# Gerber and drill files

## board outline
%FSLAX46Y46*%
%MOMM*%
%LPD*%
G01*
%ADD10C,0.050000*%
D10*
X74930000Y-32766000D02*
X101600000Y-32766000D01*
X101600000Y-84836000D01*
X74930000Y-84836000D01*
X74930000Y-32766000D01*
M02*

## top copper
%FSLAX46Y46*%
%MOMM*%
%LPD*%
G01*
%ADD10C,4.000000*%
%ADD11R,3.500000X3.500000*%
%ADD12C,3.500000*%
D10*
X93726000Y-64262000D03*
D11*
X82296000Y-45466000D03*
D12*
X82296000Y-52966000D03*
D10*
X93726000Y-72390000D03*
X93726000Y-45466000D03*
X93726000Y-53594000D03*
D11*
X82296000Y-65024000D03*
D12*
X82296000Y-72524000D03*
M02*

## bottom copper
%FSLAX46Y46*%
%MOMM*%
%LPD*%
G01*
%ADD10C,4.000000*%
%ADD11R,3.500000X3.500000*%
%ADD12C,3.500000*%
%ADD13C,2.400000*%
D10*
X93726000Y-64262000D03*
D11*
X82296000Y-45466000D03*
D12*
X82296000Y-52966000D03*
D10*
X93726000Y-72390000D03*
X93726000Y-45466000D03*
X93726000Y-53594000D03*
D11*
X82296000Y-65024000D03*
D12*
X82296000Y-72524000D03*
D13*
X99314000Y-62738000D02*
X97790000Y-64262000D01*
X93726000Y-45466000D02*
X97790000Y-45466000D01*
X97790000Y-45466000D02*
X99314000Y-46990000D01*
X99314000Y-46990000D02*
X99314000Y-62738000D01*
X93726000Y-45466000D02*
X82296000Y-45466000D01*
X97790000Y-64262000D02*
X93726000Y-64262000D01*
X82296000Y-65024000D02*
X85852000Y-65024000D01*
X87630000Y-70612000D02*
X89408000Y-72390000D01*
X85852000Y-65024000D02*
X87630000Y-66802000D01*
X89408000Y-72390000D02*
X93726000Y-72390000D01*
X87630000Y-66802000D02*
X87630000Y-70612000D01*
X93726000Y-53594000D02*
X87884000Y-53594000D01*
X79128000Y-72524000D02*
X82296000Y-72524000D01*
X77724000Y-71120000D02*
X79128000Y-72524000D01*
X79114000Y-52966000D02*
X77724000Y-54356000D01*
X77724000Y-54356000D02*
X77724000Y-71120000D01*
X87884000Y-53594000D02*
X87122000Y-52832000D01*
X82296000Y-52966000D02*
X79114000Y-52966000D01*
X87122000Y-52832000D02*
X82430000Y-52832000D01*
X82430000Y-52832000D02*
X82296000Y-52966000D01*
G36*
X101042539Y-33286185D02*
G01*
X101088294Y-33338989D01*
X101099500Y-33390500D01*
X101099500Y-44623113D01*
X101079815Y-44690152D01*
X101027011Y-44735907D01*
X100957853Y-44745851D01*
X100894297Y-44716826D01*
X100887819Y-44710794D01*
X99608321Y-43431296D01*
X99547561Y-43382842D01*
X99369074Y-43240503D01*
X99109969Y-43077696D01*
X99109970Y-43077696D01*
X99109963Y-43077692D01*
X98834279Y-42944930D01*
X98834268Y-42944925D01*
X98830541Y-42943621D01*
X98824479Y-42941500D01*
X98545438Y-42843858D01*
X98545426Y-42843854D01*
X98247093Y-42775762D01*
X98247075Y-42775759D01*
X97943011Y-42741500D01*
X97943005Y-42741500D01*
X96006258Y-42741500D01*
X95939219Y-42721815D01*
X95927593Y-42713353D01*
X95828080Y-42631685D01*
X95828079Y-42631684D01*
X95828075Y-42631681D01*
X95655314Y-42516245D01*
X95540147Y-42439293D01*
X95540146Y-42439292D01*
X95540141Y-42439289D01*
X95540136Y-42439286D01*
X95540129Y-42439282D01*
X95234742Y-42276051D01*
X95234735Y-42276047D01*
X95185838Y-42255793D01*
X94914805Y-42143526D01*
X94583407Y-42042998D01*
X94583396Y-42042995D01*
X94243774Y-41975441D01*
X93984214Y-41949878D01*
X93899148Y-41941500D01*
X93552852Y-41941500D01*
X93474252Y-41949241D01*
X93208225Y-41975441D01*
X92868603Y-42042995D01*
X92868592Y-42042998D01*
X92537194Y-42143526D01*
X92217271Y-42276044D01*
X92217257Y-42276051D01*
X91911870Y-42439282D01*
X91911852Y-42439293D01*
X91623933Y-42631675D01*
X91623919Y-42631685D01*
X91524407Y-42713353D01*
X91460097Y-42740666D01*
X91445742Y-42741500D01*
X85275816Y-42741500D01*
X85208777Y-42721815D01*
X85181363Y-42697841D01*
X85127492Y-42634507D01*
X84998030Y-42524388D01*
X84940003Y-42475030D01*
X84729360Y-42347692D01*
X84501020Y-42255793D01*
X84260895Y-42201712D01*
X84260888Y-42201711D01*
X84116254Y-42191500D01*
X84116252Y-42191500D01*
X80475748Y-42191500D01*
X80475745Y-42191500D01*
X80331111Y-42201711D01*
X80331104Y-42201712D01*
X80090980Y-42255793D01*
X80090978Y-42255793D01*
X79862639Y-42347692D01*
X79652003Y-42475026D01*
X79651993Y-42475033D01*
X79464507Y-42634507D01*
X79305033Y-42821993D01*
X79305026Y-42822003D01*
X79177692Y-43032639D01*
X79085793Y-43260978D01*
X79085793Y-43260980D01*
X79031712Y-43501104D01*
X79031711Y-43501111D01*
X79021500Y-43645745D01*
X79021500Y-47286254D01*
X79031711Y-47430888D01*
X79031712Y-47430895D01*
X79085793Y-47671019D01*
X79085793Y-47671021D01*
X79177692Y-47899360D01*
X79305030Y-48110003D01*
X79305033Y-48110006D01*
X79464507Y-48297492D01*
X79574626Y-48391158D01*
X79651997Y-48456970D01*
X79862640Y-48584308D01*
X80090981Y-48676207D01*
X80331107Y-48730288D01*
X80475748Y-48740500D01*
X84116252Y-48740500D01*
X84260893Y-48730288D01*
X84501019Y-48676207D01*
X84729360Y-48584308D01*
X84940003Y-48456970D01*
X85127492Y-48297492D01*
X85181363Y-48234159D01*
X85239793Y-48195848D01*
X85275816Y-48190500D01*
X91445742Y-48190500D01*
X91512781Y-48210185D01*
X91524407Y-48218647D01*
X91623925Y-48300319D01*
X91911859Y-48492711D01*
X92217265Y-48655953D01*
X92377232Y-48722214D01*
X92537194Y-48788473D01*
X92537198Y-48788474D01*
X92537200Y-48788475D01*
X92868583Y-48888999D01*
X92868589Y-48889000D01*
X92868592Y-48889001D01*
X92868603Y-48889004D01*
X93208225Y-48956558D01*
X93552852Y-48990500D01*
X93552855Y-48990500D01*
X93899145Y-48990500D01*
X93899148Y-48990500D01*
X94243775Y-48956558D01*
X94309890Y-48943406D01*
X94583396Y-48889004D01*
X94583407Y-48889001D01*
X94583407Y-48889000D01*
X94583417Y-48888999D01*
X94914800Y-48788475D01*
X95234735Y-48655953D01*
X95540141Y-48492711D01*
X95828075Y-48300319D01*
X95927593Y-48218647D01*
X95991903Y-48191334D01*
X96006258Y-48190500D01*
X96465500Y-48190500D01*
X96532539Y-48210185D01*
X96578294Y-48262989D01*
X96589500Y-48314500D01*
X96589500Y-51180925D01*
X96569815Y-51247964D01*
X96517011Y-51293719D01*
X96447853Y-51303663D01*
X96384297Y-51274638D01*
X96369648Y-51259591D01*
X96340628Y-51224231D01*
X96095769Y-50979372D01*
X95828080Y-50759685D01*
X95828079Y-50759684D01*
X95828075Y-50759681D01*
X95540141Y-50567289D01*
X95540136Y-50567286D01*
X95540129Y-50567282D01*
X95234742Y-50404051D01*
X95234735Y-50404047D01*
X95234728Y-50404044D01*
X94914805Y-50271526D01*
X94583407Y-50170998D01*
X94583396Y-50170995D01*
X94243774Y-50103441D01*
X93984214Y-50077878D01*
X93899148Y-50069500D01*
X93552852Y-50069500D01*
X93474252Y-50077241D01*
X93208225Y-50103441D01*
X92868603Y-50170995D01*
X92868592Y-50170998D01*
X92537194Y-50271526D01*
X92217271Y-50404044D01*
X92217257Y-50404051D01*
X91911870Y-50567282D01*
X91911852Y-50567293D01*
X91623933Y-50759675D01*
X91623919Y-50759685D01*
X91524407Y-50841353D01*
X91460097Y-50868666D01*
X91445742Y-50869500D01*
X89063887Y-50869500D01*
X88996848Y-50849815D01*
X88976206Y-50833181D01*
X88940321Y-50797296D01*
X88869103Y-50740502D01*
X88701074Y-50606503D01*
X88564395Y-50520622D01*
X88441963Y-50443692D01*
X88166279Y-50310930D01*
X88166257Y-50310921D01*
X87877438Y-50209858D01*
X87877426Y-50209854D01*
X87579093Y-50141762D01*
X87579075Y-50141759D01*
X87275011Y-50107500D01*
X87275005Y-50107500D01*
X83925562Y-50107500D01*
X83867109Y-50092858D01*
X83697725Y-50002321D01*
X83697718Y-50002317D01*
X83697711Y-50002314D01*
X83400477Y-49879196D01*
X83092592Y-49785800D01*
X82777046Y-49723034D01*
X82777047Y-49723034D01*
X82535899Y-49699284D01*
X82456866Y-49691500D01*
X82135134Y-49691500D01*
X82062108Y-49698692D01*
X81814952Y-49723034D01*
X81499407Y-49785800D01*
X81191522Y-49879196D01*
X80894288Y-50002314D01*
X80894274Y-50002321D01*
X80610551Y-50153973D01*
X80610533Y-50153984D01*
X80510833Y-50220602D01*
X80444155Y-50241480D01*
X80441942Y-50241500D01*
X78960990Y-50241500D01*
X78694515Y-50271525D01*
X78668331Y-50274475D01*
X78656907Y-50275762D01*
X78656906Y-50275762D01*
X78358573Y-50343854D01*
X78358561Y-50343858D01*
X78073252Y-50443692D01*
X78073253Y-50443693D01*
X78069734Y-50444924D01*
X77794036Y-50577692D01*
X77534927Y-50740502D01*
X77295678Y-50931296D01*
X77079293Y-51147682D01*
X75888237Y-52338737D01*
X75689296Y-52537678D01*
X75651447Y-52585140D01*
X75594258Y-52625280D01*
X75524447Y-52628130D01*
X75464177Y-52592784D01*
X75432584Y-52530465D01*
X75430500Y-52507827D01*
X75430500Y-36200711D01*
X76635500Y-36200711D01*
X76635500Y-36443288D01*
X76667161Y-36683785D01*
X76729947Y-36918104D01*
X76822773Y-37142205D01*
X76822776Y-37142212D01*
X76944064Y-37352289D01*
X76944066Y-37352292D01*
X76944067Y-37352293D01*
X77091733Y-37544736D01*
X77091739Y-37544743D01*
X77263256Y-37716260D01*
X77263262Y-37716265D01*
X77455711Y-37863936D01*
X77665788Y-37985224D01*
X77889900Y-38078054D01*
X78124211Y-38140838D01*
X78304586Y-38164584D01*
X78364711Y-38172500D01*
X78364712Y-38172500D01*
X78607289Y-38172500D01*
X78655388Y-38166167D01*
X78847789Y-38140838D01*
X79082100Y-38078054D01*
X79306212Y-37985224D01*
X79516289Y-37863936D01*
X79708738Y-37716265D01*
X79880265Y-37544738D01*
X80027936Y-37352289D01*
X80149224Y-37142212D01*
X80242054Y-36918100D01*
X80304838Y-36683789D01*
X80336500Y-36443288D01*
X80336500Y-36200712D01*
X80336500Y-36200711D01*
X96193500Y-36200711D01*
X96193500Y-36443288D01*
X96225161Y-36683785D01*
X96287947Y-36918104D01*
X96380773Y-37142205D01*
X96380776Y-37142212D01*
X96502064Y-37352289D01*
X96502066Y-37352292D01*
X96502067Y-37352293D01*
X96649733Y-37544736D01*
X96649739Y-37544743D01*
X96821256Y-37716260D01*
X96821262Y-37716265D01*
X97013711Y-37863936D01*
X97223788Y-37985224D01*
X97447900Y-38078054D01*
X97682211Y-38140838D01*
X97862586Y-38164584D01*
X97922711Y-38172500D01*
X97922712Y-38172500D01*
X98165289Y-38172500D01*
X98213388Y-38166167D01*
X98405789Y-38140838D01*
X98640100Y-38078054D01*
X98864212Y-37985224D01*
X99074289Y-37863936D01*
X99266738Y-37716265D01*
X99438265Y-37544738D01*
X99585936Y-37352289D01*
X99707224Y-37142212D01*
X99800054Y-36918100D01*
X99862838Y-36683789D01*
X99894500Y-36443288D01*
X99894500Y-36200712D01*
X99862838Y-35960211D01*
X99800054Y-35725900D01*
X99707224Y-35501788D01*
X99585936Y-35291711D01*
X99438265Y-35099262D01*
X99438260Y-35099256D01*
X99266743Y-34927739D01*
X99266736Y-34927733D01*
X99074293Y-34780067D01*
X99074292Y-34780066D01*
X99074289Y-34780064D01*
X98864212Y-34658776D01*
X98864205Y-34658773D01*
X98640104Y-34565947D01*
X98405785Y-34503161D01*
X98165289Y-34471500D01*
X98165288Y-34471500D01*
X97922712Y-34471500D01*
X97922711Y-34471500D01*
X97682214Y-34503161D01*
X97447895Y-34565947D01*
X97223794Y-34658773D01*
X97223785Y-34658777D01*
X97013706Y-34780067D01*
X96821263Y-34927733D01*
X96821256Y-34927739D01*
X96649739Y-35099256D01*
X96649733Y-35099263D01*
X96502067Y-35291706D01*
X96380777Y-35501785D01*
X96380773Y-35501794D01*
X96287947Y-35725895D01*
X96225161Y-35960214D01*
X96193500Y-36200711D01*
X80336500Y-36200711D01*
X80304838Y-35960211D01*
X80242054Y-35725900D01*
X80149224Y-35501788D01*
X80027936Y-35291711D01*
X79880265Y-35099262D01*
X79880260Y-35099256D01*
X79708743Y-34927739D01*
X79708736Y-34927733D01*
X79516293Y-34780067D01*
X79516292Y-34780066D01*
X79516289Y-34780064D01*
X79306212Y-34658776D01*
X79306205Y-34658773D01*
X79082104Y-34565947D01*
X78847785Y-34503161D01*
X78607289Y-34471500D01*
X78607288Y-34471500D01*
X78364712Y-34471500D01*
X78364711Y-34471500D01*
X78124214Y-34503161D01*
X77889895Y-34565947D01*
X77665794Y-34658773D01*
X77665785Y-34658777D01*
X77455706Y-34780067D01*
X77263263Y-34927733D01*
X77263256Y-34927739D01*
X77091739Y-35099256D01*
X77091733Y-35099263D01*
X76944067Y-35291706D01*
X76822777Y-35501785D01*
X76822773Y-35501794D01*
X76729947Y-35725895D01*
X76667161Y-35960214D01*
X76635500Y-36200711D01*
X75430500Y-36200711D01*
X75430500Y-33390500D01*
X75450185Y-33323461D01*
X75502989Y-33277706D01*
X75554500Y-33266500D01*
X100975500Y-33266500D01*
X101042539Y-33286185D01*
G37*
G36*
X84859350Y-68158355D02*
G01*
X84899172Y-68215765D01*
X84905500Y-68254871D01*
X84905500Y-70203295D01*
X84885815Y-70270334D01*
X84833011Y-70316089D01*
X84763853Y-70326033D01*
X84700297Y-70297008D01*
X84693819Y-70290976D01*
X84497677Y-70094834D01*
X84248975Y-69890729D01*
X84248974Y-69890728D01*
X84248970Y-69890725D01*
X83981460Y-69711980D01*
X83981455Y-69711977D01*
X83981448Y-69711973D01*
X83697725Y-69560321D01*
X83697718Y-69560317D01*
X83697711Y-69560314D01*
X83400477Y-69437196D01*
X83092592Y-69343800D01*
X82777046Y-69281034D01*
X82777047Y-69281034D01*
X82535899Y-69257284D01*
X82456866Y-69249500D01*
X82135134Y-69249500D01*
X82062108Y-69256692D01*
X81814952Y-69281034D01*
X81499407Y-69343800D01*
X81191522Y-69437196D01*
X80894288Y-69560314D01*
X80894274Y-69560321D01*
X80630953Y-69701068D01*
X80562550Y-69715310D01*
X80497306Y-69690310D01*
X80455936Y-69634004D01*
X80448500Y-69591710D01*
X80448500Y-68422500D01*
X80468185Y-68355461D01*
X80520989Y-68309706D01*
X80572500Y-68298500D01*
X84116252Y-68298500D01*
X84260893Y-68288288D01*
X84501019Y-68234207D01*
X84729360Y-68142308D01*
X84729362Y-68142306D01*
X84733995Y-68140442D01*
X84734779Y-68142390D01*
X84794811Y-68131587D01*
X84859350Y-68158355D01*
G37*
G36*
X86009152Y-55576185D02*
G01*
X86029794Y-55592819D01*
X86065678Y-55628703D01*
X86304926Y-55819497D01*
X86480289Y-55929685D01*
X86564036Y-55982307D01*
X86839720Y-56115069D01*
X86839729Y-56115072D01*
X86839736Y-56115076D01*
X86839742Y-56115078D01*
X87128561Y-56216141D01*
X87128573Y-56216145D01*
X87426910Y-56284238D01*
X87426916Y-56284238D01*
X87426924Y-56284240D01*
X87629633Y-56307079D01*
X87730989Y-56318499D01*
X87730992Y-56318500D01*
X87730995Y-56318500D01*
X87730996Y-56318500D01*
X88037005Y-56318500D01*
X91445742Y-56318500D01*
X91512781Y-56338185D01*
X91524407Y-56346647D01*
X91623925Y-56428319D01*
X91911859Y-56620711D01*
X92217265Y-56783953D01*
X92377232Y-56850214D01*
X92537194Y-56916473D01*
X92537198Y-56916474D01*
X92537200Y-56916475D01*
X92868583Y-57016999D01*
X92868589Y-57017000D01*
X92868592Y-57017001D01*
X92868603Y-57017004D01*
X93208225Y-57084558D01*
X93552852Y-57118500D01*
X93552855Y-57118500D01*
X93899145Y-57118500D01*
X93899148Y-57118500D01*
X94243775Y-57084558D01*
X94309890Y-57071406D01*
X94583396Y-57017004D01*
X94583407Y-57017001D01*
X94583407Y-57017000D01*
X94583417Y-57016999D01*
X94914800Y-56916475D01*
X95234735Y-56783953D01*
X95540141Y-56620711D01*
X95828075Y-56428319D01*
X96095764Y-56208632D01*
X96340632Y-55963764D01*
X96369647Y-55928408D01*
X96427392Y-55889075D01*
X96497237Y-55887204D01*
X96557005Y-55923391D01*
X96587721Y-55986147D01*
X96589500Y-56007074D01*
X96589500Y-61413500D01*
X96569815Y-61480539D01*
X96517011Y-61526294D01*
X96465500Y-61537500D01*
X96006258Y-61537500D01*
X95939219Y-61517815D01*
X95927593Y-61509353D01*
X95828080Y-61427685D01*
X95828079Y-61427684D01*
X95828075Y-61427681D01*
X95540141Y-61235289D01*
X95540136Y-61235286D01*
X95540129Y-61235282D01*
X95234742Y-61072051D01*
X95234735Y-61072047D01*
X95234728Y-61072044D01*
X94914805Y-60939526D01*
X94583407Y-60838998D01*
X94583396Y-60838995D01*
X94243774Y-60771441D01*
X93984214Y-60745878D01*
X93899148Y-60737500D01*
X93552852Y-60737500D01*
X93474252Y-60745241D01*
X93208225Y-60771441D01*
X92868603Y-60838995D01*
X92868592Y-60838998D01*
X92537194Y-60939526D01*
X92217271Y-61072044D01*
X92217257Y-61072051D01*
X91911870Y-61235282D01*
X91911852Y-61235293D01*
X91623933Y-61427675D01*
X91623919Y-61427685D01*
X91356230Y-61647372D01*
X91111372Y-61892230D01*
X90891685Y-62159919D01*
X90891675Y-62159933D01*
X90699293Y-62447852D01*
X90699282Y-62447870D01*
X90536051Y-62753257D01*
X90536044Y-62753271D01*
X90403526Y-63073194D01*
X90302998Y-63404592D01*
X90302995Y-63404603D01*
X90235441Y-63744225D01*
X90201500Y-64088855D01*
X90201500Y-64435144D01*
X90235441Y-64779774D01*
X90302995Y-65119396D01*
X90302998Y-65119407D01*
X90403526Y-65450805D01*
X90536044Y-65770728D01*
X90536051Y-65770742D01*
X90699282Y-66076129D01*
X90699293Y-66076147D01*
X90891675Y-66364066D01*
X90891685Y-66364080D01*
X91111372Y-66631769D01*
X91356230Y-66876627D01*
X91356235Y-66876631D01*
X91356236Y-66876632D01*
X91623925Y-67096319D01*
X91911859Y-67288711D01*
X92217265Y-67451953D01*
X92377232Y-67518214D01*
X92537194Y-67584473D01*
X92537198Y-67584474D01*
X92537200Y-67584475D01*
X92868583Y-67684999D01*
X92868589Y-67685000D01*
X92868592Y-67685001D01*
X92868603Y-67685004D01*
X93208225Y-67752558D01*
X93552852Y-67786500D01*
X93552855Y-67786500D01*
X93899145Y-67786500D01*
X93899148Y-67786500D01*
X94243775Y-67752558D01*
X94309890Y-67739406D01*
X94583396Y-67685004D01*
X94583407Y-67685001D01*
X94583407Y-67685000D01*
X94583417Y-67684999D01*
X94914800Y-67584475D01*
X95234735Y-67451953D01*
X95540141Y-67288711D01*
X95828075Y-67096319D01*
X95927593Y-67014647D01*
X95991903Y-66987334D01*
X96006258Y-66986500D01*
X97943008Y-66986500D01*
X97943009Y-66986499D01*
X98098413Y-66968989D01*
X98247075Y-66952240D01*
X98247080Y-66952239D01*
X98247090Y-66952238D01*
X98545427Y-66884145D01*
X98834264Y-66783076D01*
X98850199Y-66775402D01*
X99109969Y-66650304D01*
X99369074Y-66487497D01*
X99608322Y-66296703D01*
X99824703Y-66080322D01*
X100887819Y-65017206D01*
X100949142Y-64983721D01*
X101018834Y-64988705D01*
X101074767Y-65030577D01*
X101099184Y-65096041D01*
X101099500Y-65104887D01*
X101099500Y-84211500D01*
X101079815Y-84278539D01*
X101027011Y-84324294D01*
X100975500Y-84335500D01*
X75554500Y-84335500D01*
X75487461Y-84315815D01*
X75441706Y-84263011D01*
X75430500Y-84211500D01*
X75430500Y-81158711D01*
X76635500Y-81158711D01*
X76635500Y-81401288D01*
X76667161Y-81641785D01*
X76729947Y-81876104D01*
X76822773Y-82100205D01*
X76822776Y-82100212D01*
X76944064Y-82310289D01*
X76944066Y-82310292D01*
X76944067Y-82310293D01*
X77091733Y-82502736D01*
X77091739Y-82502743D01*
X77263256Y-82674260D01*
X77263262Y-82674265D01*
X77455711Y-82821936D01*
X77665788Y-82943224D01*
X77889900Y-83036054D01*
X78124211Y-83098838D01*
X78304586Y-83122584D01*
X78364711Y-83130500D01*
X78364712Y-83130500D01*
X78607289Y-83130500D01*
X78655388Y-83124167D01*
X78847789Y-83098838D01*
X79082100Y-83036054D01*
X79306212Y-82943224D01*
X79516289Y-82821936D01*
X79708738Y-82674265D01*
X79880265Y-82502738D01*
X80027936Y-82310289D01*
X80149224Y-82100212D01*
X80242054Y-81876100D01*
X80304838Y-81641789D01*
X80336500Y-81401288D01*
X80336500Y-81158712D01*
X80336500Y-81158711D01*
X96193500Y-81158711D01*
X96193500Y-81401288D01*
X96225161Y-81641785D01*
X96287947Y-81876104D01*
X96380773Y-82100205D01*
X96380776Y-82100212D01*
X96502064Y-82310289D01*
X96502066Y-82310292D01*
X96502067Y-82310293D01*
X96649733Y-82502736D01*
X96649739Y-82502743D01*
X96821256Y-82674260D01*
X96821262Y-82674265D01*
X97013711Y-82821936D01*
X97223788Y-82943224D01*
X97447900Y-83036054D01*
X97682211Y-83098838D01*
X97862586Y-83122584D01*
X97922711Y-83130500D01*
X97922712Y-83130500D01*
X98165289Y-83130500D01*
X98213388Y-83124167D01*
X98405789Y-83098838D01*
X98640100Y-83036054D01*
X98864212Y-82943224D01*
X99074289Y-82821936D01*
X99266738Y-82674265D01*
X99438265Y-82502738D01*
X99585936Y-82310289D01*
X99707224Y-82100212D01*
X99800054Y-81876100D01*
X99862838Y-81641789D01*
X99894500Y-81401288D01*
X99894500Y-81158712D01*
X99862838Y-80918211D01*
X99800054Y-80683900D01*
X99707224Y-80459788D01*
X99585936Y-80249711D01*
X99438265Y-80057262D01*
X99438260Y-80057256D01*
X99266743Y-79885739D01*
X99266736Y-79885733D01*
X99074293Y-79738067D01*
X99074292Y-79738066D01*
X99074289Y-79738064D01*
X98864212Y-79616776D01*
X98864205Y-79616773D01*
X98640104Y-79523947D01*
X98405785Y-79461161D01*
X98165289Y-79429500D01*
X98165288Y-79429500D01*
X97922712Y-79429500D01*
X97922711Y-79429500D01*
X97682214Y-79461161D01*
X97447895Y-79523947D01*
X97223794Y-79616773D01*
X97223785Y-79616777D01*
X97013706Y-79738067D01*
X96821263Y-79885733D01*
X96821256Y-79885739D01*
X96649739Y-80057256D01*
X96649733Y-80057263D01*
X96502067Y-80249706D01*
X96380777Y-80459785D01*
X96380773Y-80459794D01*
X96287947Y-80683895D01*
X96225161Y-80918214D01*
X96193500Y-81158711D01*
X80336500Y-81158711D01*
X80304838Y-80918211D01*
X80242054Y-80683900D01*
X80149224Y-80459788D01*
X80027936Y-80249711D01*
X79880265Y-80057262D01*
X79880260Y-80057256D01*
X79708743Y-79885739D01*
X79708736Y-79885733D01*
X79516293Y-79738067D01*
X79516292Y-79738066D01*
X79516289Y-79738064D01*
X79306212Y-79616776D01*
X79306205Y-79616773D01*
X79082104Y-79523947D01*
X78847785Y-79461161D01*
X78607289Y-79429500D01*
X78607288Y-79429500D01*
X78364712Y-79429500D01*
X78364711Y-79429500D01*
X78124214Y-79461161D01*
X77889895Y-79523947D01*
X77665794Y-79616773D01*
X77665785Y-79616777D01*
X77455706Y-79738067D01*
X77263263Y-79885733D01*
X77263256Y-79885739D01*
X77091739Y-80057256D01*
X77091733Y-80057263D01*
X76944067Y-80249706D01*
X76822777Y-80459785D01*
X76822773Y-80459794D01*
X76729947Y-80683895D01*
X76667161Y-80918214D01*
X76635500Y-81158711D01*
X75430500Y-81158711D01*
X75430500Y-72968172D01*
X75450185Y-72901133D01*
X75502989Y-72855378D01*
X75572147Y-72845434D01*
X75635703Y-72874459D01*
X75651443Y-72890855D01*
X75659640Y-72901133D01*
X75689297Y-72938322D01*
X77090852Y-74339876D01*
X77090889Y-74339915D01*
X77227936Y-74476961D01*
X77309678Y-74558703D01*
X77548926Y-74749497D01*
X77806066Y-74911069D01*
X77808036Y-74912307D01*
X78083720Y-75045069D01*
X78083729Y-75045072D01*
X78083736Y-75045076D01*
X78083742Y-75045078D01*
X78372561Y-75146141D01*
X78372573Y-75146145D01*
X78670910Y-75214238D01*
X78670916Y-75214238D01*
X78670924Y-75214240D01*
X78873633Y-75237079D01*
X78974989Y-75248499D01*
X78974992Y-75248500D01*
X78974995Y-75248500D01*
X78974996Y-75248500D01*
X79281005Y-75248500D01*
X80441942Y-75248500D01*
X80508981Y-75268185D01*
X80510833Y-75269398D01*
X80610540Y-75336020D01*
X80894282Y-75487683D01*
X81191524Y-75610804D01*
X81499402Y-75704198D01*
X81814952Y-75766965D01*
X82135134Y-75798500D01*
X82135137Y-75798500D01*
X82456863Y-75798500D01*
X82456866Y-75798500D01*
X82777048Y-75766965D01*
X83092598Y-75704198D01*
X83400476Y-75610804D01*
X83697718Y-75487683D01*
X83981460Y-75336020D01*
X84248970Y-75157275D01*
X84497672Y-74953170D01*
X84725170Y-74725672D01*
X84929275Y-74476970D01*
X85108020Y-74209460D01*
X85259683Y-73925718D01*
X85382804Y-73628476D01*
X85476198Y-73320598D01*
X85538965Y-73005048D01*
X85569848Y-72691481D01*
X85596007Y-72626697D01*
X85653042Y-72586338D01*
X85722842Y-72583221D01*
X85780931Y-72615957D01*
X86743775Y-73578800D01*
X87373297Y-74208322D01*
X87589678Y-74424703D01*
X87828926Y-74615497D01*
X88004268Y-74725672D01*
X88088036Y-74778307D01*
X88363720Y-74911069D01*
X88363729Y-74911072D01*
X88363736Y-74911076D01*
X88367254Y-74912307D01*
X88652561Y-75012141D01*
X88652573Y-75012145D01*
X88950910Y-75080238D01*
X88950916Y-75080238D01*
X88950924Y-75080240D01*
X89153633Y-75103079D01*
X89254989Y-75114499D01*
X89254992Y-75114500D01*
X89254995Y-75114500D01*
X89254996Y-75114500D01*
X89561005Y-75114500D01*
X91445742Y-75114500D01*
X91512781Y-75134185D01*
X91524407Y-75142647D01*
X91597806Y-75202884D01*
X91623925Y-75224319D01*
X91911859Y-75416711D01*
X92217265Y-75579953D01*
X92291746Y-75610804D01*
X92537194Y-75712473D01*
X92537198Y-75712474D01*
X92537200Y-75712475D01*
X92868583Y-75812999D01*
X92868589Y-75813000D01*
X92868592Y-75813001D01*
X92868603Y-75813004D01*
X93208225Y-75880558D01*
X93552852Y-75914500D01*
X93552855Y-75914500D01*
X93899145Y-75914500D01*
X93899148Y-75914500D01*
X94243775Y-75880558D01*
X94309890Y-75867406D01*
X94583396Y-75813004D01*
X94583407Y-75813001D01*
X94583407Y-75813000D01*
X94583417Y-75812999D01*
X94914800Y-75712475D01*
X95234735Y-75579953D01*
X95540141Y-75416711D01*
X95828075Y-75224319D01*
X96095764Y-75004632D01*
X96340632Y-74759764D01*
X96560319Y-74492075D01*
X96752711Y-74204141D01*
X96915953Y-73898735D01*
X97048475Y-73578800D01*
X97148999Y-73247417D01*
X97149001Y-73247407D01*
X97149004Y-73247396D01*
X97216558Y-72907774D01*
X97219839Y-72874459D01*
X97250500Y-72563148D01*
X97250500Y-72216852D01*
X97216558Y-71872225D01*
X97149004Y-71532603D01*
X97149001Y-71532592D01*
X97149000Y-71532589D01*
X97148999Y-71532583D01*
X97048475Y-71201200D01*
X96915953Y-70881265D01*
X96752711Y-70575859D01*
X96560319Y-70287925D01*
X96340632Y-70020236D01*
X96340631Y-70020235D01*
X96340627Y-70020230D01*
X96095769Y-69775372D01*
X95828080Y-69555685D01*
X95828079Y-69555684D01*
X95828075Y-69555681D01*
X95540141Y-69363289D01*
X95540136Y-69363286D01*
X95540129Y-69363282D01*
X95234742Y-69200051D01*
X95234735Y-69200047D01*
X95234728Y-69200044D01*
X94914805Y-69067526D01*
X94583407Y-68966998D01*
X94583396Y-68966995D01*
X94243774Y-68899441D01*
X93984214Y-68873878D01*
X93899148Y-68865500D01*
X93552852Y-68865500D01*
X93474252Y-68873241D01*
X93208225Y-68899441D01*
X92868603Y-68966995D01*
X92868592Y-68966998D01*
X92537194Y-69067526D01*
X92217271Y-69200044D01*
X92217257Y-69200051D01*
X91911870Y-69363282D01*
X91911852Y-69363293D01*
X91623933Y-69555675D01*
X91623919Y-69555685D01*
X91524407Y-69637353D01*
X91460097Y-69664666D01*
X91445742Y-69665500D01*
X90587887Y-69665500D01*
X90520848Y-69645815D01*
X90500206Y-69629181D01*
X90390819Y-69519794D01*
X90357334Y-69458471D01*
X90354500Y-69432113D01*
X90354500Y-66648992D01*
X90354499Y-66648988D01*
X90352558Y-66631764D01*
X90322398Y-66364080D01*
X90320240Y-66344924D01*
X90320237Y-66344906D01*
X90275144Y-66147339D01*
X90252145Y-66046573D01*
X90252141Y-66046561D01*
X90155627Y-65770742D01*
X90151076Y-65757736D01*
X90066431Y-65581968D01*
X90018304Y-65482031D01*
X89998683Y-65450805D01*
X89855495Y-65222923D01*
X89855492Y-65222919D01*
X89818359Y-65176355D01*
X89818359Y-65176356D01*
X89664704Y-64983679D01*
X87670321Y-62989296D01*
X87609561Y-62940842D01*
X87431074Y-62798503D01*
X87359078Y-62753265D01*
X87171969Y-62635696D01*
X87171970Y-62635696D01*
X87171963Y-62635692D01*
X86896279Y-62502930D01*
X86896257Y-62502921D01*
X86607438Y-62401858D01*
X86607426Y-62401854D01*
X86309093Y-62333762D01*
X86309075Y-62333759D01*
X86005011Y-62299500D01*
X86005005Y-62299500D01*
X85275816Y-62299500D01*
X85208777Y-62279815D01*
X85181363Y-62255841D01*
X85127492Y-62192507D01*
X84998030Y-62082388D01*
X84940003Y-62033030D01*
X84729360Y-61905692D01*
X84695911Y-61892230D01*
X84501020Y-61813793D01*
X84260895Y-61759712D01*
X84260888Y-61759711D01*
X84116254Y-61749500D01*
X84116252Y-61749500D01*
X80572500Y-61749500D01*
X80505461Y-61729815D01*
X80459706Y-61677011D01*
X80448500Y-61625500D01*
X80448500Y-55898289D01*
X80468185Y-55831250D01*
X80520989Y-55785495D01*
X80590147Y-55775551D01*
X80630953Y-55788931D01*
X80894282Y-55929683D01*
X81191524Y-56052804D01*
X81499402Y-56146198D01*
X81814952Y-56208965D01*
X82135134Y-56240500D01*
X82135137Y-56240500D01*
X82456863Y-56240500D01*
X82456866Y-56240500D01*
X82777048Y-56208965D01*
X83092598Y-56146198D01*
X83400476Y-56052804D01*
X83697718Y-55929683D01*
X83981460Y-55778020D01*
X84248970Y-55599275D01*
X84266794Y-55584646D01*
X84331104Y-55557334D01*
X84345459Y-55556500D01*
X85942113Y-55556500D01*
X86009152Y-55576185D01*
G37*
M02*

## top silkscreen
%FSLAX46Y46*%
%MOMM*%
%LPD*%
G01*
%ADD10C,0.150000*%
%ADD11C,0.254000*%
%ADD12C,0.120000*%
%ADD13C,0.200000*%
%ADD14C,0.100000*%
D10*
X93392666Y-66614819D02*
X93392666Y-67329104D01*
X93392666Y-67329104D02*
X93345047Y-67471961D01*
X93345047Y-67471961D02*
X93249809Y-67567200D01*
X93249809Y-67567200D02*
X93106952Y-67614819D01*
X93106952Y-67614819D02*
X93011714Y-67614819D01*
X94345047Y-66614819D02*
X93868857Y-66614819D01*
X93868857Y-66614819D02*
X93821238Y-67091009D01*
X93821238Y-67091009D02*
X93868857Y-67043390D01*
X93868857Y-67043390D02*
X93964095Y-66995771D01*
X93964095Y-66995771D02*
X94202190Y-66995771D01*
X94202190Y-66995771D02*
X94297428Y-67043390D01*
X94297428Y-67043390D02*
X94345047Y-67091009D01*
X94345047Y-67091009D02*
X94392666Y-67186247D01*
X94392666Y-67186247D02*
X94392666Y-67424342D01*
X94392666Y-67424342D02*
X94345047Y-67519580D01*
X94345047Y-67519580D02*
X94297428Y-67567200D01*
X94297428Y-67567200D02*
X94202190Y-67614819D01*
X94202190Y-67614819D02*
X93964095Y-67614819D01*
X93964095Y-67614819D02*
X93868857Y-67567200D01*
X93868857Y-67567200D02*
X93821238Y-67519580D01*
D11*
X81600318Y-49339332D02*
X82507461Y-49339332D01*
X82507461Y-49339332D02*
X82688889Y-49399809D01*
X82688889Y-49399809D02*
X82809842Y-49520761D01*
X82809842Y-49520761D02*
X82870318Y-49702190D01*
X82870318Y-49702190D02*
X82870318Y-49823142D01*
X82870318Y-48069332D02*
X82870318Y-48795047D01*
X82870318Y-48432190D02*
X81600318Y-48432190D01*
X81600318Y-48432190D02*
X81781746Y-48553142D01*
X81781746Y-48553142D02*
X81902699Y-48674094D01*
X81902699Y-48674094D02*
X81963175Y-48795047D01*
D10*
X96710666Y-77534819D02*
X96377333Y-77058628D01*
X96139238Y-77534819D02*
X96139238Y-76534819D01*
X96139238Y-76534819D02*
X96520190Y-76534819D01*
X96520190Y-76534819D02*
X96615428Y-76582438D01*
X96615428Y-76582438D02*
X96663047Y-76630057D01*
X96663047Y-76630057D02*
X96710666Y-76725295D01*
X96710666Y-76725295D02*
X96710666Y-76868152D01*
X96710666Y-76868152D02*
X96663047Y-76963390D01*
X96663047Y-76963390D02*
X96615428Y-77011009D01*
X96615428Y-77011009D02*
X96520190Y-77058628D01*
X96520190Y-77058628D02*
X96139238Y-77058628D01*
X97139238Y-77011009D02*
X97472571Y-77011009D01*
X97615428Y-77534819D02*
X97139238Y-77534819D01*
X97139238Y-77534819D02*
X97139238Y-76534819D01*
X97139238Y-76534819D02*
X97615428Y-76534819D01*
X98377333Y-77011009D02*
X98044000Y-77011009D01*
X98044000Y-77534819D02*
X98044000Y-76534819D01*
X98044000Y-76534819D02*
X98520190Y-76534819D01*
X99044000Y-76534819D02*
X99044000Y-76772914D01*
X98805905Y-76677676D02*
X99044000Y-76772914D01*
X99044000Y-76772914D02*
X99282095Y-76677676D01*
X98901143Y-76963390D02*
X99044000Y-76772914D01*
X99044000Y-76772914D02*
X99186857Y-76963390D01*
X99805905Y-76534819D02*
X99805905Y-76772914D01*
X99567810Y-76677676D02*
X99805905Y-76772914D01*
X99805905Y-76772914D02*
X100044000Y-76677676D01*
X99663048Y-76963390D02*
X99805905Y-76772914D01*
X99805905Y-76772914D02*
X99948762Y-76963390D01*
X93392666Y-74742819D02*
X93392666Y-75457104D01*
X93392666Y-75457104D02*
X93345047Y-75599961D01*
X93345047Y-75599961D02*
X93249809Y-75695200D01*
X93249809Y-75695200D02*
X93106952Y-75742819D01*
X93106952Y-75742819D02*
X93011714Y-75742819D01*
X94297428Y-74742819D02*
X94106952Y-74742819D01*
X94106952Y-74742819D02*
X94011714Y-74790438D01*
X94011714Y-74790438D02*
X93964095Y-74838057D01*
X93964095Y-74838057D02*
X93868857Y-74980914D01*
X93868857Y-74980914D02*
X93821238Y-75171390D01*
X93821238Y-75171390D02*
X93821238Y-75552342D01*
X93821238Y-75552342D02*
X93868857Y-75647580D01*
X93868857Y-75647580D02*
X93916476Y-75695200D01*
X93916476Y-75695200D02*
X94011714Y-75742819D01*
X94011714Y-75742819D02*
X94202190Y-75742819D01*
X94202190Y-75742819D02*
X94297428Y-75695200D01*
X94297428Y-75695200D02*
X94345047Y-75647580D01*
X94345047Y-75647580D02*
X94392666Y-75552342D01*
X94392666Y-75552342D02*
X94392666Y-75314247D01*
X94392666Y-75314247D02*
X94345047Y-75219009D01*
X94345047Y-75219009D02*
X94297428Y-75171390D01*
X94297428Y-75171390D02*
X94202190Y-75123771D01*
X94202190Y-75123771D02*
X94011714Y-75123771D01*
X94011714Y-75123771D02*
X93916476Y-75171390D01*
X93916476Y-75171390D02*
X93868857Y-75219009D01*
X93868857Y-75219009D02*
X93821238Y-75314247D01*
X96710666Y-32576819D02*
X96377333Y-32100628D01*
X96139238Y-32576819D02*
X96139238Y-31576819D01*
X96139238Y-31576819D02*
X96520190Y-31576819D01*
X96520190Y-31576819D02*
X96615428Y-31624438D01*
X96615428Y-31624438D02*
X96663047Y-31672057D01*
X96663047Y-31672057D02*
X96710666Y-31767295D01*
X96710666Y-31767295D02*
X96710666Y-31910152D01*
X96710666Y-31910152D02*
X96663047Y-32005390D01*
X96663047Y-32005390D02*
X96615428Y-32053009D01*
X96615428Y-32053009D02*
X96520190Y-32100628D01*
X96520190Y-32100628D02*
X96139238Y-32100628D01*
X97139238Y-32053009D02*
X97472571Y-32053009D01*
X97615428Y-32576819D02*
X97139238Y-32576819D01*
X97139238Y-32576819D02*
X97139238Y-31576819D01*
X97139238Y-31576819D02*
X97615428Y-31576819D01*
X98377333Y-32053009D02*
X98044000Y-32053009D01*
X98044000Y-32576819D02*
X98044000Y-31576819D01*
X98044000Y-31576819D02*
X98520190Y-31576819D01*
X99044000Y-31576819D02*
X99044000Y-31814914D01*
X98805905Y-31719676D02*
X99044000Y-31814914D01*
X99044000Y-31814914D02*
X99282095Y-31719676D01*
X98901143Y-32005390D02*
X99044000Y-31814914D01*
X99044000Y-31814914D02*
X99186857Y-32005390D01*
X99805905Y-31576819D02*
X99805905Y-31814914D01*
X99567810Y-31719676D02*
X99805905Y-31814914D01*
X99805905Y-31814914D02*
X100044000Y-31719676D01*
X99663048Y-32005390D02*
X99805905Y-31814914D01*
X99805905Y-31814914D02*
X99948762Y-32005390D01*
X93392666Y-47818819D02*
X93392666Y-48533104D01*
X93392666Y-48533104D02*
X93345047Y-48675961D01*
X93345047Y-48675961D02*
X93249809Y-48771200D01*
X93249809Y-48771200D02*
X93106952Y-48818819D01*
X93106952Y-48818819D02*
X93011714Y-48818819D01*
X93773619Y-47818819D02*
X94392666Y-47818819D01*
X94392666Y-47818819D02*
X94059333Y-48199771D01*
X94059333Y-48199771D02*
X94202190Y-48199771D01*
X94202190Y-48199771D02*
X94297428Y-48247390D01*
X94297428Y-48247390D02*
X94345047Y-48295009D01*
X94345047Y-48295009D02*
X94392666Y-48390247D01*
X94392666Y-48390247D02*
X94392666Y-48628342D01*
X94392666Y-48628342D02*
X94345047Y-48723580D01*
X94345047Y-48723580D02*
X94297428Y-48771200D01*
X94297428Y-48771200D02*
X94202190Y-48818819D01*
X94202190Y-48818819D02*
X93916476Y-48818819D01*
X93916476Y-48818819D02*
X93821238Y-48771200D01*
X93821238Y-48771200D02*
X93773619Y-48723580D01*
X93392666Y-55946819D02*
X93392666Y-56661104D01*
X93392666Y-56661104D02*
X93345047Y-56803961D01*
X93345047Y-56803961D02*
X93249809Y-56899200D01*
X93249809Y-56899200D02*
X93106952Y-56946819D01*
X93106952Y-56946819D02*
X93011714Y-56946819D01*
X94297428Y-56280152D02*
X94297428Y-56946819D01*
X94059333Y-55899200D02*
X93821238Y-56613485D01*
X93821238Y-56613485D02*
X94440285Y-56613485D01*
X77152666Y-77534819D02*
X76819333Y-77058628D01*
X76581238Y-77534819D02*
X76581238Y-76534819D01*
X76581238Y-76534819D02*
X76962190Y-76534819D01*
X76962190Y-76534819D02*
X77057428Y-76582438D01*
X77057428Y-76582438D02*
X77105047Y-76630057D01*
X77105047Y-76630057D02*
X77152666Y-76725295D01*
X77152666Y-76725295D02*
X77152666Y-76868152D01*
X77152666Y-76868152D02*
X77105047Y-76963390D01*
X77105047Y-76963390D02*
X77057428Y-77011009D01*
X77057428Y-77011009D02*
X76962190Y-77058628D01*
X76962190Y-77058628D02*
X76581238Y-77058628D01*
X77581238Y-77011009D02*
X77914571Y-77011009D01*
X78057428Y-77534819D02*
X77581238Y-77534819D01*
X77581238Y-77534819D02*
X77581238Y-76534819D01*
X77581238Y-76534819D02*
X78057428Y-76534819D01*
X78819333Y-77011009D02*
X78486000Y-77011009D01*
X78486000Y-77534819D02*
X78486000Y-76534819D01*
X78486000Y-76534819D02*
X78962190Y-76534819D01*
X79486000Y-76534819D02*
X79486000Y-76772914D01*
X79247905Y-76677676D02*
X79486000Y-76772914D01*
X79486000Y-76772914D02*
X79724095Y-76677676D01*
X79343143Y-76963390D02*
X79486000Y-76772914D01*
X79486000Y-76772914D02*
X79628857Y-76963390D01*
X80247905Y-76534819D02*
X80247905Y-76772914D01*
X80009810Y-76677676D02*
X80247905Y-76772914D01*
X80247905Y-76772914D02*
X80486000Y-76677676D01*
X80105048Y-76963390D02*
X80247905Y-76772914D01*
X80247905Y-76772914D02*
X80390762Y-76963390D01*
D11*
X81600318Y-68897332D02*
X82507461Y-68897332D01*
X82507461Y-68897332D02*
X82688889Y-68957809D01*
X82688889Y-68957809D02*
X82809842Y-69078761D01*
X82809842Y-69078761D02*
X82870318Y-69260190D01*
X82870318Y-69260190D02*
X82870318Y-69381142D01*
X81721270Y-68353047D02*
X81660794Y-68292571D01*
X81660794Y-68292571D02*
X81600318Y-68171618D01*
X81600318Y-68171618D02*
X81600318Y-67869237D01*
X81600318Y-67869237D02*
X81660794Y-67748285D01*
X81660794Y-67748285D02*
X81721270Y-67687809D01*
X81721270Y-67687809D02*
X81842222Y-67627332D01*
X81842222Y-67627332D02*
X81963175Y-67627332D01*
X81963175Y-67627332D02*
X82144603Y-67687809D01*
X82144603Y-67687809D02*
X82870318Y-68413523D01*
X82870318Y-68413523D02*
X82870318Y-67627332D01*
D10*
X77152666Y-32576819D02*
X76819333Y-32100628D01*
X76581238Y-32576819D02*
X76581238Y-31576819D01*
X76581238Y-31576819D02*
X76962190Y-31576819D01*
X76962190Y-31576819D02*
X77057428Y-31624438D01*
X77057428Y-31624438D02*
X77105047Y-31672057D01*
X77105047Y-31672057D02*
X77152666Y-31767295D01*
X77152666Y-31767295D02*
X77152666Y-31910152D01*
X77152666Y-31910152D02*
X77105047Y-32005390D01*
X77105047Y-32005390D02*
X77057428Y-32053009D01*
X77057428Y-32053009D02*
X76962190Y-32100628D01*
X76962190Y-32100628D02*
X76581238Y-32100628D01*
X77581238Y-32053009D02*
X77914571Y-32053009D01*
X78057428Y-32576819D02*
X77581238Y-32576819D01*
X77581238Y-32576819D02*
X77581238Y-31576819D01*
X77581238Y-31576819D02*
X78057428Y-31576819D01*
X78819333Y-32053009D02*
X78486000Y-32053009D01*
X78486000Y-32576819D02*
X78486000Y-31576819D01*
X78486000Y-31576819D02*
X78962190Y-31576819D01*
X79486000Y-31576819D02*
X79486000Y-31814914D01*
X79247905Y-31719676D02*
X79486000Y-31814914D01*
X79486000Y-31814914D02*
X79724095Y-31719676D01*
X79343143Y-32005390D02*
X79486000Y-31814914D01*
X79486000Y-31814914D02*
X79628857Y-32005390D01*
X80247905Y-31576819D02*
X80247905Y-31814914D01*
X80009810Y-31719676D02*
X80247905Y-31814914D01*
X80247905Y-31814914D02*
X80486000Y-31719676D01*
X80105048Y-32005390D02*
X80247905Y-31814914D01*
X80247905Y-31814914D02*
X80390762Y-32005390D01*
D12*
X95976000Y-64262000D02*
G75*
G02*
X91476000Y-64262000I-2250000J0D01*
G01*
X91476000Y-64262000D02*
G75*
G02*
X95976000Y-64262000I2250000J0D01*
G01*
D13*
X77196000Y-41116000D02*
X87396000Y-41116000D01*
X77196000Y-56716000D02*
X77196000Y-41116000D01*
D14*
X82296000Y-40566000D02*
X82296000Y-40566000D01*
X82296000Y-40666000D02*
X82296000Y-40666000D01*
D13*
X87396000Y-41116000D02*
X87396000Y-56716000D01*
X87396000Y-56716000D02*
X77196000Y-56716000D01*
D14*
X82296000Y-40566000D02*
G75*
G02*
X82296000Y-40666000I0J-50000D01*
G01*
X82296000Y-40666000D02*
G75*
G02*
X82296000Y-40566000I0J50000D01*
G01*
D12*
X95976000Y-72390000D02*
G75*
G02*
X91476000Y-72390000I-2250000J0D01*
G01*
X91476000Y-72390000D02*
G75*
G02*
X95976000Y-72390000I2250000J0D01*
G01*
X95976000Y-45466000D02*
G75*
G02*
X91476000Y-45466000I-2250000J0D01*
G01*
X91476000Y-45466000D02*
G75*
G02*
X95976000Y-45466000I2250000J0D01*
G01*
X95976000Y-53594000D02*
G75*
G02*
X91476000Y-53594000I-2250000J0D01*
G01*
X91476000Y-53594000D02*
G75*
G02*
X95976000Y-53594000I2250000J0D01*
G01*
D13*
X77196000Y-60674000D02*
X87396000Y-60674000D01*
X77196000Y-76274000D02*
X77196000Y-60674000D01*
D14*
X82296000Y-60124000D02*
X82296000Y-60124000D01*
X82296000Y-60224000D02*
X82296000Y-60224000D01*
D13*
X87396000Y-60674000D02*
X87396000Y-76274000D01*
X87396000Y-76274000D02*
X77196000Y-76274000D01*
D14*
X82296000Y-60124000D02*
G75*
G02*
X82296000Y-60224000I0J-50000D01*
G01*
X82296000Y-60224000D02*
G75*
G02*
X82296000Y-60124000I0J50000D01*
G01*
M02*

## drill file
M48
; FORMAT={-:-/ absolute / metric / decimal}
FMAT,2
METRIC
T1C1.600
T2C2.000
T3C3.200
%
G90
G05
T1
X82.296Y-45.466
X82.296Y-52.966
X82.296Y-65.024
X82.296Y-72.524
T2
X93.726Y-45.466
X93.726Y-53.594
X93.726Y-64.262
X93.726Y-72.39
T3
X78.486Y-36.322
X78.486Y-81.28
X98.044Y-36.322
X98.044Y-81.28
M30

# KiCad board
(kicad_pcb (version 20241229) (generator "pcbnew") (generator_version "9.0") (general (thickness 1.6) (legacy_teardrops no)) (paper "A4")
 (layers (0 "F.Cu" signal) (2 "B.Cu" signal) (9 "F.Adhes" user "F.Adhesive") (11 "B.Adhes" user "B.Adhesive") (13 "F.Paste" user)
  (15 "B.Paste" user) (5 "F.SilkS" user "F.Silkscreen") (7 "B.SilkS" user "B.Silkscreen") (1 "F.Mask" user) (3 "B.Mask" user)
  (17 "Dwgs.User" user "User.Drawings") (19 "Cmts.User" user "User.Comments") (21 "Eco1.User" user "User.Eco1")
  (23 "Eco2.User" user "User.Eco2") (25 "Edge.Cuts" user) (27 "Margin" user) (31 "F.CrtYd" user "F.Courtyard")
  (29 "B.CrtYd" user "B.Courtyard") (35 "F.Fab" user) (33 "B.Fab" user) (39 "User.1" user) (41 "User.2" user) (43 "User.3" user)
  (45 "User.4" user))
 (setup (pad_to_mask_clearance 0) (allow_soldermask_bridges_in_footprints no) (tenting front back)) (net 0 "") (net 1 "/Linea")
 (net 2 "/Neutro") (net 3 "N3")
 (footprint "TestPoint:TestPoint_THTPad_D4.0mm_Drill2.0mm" (layer "F.Cu") (at 93.726 64.262 180)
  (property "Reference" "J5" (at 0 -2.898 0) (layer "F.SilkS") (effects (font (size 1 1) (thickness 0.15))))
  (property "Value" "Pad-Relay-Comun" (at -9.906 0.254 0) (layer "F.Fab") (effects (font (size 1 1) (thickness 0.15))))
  (fp_circle (center 0 0) (end 0 2.25) (stroke (width 0.12) (type solid)) (fill no) (layer "F.SilkS"))
  (pad "1" thru_hole circle (at 0 0 180) (size 4 4) (drill 2) (layers "*.Cu" "*.Mask") (remove_unused_layers no) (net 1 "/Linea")))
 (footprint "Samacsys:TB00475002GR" (layer "F.Cu") (at 82.296 45.466 -90)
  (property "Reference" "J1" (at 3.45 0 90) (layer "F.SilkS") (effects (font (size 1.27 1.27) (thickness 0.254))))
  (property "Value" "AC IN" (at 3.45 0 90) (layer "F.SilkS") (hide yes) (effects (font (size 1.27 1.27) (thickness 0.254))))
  (fp_line (start -4.35 5.1) (end -4.35 -5.1) (stroke (width 0.2) (type solid)) (layer "F.SilkS"))
  (fp_line (start 11.25 5.1) (end -4.35 5.1) (stroke (width 0.2) (type solid)) (layer "F.SilkS"))
  (fp_line (start -4.9 0) (end -4.9 0) (stroke (width 0.1) (type solid)) (layer "F.SilkS"))
  (fp_line (start -4.8 0) (end -4.8 0) (stroke (width 0.1) (type solid)) (layer "F.SilkS"))
  (fp_line (start -4.35 -5.1) (end 11.25 -5.1) (stroke (width 0.2) (type solid)) (layer "F.SilkS"))
  (fp_line (start 11.25 -5.1) (end 11.25 5.1) (stroke (width 0.2) (type solid)) (layer "F.SilkS"))
  (fp_arc (start -4.9 0) (mid -4.85 -0.05) (end -4.8 0) (stroke (width 0.1) (type solid)) (layer "F.SilkS"))
  (fp_arc (start -4.8 0) (mid -4.85 0.05) (end -4.9 0) (stroke (width 0.1) (type solid)) (layer "F.SilkS"))
  (pad "1" thru_hole rect (at 0 0 270) (size 3.5 3.5) (drill 1.6) (layers "*.Cu" "*.Mask") (remove_unused_layers no) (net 1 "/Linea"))
  (pad "2" thru_hole circle (at 7.5 0 270) (size 3.5 3.5) (drill 1.6) (layers "*.Cu" "*.Mask") (remove_unused_layers no) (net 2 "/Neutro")))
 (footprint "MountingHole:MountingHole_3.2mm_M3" (layer "F.Cu") (at 98.044 81.28)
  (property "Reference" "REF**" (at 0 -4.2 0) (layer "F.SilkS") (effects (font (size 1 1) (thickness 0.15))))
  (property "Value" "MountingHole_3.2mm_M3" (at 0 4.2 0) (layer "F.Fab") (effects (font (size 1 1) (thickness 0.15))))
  (pad "" np_thru_hole circle (at 0 0) (size 3.2 3.2) (drill 3.2) (layers "*.Cu" "*.Mask")))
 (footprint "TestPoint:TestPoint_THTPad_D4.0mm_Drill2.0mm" (layer "F.Cu") (at 93.726 72.39 180)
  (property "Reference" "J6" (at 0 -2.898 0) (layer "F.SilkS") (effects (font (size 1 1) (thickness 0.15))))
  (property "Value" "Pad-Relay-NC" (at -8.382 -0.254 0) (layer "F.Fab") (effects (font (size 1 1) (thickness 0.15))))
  (fp_circle (center 0 0) (end 0 2.25) (stroke (width 0.12) (type solid)) (fill no) (layer "F.SilkS"))
  (pad "1" thru_hole circle (at 0 0 180) (size 4 4) (drill 2) (layers "*.Cu" "*.Mask") (remove_unused_layers no) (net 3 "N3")))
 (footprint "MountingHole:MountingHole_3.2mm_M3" (layer "F.Cu") (at 98.044 36.322)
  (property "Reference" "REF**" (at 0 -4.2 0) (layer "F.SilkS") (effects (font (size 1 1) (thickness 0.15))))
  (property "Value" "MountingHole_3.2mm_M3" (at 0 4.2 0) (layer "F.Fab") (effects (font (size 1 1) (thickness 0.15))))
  (pad "" np_thru_hole circle (at 0 0) (size 3.2 3.2) (drill 3.2) (layers "*.Cu" "*.Mask")))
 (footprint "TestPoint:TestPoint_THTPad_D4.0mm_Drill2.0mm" (layer "F.Cu") (at 93.726 45.466 180)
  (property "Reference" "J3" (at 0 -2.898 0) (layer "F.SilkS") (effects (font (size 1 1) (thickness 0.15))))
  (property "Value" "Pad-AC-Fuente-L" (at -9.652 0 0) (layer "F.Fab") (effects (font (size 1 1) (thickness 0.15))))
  (fp_circle (center 0 0) (end 0 2.25) (stroke (width 0.12) (type solid)) (fill no) (layer "F.SilkS"))
  (pad "1" thru_hole circle (at 0 0 180) (size 4 4) (drill 2) (layers "*.Cu" "*.Mask") (remove_unused_layers no) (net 1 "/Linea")))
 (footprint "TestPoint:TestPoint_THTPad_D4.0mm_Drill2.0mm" (layer "F.Cu") (at 93.726 53.594 180)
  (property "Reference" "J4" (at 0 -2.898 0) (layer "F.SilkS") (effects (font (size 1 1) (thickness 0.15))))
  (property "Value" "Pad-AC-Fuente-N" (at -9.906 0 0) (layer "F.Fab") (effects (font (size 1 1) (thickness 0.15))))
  (fp_circle (center 0 0) (end 0 2.25) (stroke (width 0.12) (type solid)) (fill no) (layer "F.SilkS"))
  (pad "1" thru_hole circle (at 0 0 180) (size 4 4) (drill 2) (layers "*.Cu" "*.Mask") (remove_unused_layers no) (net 2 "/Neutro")))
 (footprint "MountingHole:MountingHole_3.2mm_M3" (layer "F.Cu") (at 78.486 81.28)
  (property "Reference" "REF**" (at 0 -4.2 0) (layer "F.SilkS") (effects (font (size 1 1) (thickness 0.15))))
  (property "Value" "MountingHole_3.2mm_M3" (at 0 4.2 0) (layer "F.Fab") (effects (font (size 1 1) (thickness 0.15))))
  (pad "" np_thru_hole circle (at 0 0) (size 3.2 3.2) (drill 3.2) (layers "*.Cu" "*.Mask")))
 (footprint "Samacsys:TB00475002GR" (layer "F.Cu") (at 82.296 65.024 -90)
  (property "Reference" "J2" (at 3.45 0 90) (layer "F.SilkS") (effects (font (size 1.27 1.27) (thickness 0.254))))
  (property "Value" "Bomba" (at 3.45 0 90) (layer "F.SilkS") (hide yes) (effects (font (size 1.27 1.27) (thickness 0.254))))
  (fp_line (start -4.35 5.1) (end -4.35 -5.1) (stroke (width 0.2) (type solid)) (layer "F.SilkS"))
  (fp_line (start 11.25 5.1) (end -4.35 5.1) (stroke (width 0.2) (type solid)) (layer "F.SilkS"))
  (fp_line (start -4.9 0) (end -4.9 0) (stroke (width 0.1) (type solid)) (layer "F.SilkS"))
  (fp_line (start -4.8 0) (end -4.8 0) (stroke (width 0.1) (type solid)) (layer "F.SilkS"))
  (fp_line (start -4.35 -5.1) (end 11.25 -5.1) (stroke (width 0.2) (type solid)) (layer "F.SilkS"))
  (fp_line (start 11.25 -5.1) (end 11.25 5.1) (stroke (width 0.2) (type solid)) (layer "F.SilkS"))
  (fp_arc (start -4.9 0) (mid -4.85 -0.05) (end -4.8 0) (stroke (width 0.1) (type solid)) (layer "F.SilkS"))
  (fp_arc (start -4.8 0) (mid -4.85 0.05) (end -4.9 0) (stroke (width 0.1) (type solid)) (layer "F.SilkS"))
  (pad "1" thru_hole rect (at 0 0 270) (size 3.5 3.5) (drill 1.6) (layers "*.Cu" "*.Mask") (remove_unused_layers no) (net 3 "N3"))
  (pad "2" thru_hole circle (at 7.5 0 270) (size 3.5 3.5) (drill 1.6) (layers "*.Cu" "*.Mask") (remove_unused_layers no) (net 2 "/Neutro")))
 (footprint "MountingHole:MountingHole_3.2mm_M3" (layer "F.Cu") (at 78.486 36.322)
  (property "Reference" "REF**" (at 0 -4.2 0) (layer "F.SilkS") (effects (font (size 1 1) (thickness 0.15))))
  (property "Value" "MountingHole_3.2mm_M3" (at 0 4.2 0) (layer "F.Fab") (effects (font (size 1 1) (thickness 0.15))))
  (pad "" np_thru_hole circle (at 0 0) (size 3.2 3.2) (drill 3.2) (layers "*.Cu" "*.Mask")))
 (gr_rect (start 74.93 32.766) (end 101.6 84.836) (stroke (width 0.05) (type default)) (fill no) (layer "Edge.Cuts"))
 (segment (start 99.314 62.738) (end 97.79 64.262) (width 2.4) (layer "B.Cu") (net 1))
 (segment (start 93.726 45.466) (end 97.79 45.466) (width 2.4) (layer "B.Cu") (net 1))
 (segment (start 97.79 45.466) (end 99.314 46.99) (width 2.4) (layer "B.Cu") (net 1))
 (segment (start 99.314 46.99) (end 99.314 62.738) (width 2.4) (layer "B.Cu") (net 1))
 (segment (start 93.726 45.466) (end 82.296 45.466) (width 2.4) (layer "B.Cu") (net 1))
 (segment (start 97.79 64.262) (end 93.726 64.262) (width 2.4) (layer "B.Cu") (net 1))
 (segment (start 82.296 65.024) (end 85.852 65.024) (width 2.4) (layer "B.Cu") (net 3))
 (segment (start 87.63 70.612) (end 89.408 72.39) (width 2.4) (layer "B.Cu") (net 3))
 (segment (start 85.852 65.024) (end 87.63 66.802) (width 2.4) (layer "B.Cu") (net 3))
 (segment (start 89.408 72.39) (end 93.726 72.39) (width 2.4) (layer "B.Cu") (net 3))
 (segment (start 87.63 66.802) (end 87.63 70.612) (width 2.4) (layer "B.Cu") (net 3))
 (segment (start 93.726 53.594) (end 87.884 53.594) (width 2.4) (layer "B.Cu") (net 2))
 (segment (start 79.128 72.524) (end 82.296 72.524) (width 2.4) (layer "B.Cu") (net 2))
 (segment (start 77.724 71.12) (end 79.128 72.524) (width 2.4) (layer "B.Cu") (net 2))
 (segment (start 79.114 52.966) (end 77.724 54.356) (width 2.4) (layer "B.Cu") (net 2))
 (segment (start 77.724 54.356) (end 77.724 71.12) (width 2.4) (layer "B.Cu") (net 2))
 (segment (start 87.884 53.594) (end 87.122 52.832) (width 2.4) (layer "B.Cu") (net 2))
 (segment (start 82.296 52.966) (end 79.114 52.966) (width 2.4) (layer "B.Cu") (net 2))
 (segment (start 87.122 52.832) (end 82.43 52.832) (width 2.4) (layer "B.Cu") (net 2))
 (segment (start 82.43 52.832) (end 82.296 52.966) (width 2.4) (layer "B.Cu") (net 2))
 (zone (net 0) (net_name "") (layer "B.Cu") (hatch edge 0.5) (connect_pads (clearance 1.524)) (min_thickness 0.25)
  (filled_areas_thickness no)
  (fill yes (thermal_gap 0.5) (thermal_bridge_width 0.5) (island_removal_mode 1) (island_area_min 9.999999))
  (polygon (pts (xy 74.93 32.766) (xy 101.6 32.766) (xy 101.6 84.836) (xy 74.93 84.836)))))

